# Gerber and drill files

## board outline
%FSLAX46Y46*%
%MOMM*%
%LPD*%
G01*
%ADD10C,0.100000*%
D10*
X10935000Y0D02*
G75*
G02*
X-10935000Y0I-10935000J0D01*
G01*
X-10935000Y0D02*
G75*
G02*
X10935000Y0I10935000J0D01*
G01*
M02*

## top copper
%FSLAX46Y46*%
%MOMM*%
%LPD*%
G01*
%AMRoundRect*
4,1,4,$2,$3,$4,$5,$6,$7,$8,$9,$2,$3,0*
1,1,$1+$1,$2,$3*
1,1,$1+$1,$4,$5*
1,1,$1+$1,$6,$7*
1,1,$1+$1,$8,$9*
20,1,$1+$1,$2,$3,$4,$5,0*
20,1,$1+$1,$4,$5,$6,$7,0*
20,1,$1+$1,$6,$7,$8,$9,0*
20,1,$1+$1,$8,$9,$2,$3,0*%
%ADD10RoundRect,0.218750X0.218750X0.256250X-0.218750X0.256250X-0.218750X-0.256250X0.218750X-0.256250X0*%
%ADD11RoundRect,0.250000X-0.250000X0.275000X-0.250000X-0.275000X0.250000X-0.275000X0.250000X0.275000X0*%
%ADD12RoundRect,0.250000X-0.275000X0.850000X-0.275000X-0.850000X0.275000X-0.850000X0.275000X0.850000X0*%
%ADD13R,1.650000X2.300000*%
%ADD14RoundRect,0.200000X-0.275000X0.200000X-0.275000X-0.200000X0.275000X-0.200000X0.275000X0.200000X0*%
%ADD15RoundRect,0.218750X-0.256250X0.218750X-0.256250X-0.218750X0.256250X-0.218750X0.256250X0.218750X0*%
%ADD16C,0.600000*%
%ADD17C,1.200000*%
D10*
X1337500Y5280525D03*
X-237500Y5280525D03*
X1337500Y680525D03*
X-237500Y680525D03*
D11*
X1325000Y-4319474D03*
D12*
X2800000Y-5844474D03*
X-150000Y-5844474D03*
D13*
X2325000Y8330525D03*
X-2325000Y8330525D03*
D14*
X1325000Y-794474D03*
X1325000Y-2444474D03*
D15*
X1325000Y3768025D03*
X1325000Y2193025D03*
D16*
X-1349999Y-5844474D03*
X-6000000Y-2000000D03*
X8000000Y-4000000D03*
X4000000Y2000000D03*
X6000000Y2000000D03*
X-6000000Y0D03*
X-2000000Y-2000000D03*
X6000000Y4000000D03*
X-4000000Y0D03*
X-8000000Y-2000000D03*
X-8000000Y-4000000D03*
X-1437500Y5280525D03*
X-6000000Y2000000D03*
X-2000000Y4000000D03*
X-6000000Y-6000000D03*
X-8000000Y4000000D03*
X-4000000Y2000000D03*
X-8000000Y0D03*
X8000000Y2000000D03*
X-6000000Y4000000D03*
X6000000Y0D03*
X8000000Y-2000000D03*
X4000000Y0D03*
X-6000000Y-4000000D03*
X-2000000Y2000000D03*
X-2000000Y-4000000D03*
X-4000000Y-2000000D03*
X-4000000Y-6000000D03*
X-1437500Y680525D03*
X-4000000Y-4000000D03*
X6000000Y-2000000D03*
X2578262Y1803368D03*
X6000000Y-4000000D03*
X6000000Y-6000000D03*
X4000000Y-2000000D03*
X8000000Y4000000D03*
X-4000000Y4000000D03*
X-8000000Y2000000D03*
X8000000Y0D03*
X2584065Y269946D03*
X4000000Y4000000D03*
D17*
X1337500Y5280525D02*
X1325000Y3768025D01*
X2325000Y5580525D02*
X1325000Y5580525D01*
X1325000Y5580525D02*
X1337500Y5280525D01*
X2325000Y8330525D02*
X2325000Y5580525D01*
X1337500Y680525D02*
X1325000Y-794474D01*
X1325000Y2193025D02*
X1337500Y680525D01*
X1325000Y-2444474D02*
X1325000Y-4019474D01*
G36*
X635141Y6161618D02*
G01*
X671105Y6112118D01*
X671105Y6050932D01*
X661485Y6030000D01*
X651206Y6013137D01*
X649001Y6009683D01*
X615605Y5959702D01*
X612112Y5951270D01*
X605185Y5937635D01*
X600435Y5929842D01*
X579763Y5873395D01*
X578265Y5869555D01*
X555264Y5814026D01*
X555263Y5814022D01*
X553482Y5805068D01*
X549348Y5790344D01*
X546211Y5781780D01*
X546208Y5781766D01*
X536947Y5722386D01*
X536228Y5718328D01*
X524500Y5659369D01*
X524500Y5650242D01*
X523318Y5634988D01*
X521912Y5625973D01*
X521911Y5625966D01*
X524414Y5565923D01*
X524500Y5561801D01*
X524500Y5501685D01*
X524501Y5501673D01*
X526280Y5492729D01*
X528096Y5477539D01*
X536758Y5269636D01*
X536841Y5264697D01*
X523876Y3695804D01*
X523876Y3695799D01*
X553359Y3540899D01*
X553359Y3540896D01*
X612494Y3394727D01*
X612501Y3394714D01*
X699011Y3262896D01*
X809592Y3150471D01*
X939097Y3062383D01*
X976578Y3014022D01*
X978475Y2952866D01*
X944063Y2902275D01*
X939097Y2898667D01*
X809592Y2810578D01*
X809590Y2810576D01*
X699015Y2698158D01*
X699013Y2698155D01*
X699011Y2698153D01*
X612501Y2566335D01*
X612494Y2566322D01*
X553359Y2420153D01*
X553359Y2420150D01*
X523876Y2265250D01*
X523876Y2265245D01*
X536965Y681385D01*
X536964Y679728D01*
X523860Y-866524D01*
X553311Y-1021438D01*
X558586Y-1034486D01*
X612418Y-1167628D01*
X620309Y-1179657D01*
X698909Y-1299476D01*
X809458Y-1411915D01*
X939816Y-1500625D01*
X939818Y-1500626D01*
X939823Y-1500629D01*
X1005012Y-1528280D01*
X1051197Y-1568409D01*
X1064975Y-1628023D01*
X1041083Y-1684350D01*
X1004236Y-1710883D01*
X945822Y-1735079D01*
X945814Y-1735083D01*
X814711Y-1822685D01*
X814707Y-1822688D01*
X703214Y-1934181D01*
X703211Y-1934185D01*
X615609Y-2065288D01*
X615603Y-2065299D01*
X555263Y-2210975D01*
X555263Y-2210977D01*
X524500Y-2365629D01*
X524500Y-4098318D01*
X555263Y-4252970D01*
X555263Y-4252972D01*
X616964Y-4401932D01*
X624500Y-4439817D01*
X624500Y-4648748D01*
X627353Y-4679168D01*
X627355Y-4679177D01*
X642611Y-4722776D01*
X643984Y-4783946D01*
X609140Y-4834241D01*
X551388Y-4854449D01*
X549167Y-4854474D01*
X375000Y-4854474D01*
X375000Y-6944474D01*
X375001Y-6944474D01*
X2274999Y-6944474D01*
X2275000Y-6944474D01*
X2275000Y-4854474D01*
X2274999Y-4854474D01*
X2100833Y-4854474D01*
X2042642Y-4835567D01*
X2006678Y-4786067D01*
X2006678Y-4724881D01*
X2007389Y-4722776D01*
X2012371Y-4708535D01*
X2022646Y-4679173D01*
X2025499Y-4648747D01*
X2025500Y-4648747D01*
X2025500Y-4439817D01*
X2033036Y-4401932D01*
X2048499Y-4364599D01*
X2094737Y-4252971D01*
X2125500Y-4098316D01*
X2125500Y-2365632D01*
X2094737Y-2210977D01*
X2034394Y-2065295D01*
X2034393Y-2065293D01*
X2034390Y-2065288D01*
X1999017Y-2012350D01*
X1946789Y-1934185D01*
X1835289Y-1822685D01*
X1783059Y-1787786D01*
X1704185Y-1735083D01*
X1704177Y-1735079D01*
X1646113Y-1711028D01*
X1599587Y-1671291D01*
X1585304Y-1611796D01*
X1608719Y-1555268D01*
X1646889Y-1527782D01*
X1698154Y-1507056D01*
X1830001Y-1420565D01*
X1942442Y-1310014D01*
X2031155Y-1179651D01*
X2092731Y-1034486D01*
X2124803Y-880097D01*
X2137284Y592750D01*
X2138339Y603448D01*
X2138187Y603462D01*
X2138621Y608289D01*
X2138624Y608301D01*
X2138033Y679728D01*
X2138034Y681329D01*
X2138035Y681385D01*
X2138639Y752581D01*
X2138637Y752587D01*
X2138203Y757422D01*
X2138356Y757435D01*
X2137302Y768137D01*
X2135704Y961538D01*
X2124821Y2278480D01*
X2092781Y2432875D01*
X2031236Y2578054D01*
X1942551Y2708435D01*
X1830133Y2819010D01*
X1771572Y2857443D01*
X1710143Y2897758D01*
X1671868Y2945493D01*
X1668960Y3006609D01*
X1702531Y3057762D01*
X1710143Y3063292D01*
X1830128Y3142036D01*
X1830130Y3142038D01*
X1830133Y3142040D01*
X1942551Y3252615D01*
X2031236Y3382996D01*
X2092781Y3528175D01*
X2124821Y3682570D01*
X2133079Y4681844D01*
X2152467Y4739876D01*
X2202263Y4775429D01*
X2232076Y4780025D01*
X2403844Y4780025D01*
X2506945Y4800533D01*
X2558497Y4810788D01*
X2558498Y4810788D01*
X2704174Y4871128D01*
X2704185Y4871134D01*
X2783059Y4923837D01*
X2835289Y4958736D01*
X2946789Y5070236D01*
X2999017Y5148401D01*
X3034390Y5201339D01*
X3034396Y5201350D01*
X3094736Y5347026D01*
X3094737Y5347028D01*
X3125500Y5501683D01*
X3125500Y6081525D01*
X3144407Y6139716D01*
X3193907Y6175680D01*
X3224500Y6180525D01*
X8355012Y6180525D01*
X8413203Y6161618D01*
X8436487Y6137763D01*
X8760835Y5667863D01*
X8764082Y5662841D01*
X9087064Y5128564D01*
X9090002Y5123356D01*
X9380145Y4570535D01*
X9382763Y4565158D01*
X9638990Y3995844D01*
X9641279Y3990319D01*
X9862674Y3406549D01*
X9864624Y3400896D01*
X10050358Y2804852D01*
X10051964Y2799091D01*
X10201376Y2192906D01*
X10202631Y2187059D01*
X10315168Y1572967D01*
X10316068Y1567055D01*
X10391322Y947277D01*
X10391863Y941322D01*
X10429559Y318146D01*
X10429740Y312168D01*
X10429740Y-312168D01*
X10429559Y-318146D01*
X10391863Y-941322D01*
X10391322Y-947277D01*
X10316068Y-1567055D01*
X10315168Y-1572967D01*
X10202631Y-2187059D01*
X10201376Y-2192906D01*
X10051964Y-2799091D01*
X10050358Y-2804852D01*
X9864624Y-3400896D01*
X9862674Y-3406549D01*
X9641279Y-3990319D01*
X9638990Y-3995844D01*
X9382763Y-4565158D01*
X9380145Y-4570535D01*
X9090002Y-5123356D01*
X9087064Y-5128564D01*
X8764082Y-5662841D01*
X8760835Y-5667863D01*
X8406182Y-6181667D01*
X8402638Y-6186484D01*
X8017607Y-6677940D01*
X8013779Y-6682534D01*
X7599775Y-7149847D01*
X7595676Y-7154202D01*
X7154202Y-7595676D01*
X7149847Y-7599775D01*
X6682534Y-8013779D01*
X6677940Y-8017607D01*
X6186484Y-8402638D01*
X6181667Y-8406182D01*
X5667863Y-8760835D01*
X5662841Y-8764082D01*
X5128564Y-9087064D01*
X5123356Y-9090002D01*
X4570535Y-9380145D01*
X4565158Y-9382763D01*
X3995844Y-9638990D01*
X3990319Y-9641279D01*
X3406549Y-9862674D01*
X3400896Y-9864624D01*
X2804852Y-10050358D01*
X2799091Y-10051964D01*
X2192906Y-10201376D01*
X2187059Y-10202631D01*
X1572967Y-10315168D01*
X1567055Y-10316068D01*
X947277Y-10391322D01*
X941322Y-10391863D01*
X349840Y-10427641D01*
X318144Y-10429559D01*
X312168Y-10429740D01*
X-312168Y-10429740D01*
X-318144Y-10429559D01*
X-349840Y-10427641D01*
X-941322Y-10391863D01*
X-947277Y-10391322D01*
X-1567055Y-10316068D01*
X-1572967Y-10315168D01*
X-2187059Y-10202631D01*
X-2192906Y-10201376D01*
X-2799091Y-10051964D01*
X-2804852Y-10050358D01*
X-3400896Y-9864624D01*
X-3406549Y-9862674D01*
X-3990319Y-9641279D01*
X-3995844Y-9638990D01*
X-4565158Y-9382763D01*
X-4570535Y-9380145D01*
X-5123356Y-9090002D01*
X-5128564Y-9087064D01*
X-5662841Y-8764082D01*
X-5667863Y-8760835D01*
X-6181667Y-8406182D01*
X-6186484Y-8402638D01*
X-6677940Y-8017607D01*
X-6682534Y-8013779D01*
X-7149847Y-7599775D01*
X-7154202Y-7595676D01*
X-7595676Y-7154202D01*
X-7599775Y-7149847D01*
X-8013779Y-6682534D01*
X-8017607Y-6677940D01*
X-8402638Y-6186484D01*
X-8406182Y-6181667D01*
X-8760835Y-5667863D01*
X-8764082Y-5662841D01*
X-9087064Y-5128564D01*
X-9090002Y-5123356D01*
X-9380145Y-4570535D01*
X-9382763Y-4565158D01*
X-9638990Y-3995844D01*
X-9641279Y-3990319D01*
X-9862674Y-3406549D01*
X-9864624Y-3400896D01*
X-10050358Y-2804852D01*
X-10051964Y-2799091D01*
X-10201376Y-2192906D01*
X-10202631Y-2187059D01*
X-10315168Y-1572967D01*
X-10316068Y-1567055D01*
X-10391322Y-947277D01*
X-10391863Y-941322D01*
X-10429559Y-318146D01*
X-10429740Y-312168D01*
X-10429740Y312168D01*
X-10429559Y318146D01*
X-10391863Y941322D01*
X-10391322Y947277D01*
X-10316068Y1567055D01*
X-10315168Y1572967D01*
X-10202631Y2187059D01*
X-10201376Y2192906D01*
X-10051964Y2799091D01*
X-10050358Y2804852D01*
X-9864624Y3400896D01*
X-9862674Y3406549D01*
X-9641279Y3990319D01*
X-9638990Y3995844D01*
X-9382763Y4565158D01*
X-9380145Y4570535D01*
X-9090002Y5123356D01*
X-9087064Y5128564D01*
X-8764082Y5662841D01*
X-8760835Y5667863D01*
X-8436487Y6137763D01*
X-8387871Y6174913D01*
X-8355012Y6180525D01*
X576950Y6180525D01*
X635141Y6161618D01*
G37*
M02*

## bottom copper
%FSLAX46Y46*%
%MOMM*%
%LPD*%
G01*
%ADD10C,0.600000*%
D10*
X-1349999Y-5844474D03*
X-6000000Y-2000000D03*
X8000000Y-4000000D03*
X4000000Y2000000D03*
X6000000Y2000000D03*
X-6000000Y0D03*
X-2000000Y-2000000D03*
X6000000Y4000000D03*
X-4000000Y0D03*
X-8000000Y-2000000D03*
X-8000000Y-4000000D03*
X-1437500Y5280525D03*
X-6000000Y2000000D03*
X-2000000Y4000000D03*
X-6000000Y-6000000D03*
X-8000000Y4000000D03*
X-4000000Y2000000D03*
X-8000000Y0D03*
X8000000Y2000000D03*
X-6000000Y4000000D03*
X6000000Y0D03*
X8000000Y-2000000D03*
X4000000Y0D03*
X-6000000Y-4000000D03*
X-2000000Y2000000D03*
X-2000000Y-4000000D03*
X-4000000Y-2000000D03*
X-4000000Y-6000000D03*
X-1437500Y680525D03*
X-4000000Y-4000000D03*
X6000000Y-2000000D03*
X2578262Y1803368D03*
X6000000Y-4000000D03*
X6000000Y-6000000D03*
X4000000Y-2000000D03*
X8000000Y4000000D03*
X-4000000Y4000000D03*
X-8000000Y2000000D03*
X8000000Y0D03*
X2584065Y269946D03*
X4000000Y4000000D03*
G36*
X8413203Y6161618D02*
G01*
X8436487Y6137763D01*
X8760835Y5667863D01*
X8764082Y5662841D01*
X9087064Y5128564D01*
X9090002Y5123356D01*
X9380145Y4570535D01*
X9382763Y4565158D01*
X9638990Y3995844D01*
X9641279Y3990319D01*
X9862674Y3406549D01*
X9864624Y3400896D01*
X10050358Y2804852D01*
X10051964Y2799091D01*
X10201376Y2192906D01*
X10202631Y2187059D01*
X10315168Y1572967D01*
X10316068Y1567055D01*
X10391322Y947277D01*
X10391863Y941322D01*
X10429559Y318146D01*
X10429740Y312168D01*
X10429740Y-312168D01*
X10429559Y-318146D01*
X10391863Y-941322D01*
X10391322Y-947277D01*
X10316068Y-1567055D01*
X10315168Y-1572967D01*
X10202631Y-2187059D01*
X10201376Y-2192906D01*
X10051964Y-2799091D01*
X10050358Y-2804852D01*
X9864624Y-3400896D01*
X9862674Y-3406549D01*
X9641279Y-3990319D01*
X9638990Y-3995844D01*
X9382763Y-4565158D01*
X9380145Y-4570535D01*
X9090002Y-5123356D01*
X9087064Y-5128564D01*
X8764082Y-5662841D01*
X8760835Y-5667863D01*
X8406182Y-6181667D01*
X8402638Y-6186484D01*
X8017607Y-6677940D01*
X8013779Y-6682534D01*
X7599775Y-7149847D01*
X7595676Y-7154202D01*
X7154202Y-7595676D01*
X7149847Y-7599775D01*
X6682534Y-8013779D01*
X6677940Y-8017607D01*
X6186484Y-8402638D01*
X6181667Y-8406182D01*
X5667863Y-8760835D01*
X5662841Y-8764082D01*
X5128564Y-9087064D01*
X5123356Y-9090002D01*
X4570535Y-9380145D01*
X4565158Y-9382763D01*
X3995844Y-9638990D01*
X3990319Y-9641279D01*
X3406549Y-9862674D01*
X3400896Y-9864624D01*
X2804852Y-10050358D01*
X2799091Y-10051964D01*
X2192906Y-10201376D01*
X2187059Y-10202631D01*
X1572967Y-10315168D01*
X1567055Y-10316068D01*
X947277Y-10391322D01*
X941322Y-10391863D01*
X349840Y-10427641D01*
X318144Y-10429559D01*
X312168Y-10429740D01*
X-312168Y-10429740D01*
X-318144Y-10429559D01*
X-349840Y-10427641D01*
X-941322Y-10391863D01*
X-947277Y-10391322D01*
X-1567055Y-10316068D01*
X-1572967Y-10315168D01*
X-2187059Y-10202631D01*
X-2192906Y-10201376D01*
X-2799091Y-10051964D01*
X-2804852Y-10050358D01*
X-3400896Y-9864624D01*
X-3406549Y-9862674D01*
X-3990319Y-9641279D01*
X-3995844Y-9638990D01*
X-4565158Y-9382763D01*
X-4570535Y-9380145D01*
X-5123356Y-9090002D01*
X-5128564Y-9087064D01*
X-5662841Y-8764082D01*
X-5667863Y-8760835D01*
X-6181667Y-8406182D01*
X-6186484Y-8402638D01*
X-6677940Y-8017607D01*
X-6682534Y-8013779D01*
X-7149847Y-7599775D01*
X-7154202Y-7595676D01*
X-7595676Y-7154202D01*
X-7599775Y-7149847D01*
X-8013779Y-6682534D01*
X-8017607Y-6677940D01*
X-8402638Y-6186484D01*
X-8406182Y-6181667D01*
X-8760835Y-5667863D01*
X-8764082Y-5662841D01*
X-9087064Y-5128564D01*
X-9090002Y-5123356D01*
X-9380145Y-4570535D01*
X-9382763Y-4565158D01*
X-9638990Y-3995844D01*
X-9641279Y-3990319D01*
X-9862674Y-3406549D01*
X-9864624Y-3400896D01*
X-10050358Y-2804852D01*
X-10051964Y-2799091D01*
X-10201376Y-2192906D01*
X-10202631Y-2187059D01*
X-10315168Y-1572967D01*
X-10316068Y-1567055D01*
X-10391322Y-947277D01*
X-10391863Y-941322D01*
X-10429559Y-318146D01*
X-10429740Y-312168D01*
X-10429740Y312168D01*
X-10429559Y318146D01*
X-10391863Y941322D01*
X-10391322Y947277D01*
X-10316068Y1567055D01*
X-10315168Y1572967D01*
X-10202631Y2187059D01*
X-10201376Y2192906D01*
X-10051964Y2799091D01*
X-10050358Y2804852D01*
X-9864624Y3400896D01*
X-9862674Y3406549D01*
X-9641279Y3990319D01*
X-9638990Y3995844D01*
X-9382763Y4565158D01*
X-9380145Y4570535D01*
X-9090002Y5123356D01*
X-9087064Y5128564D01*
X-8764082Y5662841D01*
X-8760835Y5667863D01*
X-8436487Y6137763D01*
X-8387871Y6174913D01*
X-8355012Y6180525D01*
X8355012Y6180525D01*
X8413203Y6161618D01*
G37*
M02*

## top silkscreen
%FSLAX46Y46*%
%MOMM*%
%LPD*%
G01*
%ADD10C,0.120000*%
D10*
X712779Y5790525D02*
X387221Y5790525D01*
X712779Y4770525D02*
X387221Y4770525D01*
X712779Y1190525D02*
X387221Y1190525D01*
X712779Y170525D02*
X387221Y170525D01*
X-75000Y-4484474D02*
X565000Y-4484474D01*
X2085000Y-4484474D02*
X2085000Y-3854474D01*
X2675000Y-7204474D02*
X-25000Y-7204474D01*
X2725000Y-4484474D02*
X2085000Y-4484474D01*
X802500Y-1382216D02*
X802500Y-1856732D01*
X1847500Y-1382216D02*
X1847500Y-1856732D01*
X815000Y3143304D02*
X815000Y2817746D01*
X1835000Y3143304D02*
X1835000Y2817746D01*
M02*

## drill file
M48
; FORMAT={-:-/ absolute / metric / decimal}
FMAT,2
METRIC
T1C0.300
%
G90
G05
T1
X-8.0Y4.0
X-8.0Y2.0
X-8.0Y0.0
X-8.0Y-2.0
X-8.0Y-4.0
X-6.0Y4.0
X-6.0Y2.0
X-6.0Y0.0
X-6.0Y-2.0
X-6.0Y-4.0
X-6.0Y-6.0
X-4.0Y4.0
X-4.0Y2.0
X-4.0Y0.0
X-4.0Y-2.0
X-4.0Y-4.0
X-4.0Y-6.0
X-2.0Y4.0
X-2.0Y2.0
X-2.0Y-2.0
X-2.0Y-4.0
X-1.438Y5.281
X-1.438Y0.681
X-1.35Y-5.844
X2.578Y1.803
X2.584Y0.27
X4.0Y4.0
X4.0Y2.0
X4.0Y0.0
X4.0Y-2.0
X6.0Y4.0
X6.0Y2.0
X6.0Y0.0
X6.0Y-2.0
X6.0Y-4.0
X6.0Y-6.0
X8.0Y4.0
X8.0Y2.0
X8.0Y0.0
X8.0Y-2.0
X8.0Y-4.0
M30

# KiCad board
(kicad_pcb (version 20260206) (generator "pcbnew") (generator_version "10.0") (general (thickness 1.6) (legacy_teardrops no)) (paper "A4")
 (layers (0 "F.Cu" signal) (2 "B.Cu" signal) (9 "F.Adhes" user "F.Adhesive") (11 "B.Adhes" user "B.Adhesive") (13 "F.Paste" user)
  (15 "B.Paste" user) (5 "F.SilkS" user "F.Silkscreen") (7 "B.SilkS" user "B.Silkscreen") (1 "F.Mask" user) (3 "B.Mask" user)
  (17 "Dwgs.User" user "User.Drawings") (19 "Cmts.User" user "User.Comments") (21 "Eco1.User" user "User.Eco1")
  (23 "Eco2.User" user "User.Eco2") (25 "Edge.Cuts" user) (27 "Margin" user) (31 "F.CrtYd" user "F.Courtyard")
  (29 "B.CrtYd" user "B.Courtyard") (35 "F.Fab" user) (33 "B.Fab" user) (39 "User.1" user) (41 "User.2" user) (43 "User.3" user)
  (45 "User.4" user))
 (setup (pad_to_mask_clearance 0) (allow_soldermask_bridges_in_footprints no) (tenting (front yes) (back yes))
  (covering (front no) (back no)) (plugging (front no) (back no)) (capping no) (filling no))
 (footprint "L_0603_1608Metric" (layer "F.Cu") (at 0.55 -5.280525 180)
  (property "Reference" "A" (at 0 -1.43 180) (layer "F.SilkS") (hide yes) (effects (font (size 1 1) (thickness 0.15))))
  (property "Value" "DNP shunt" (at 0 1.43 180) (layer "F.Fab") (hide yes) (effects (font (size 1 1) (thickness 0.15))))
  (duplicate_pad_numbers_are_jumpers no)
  (fp_line (start -0.162779 0.51) (end 0.162779 0.51) (stroke (width 0.12) (type solid)) (layer "F.SilkS"))
  (fp_line (start -0.162779 -0.51) (end 0.162779 -0.51) (stroke (width 0.12) (type solid)) (layer "F.SilkS"))
  (pad "1" smd roundrect (at -0.7875 0 180) (size 0.875 0.95) (layers "F.Cu" "F.Mask" "F.Paste") (roundrect_rratio 0.25) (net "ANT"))
  (pad "2" smd roundrect (at 0.7875 0 180) (size 0.875 0.95) (layers "F.Cu" "F.Mask" "F.Paste") (roundrect_rratio 0.25) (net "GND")))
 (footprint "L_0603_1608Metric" (layer "F.Cu") (at 0.55 -0.680525 180)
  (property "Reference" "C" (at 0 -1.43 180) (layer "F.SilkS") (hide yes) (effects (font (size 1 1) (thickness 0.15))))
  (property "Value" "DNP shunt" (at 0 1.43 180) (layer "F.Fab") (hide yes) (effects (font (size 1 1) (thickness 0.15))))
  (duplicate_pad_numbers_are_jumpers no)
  (fp_line (start -0.162779 0.51) (end 0.162779 0.51) (stroke (width 0.12) (type solid)) (layer "F.SilkS"))
  (fp_line (start -0.162779 -0.51) (end 0.162779 -0.51) (stroke (width 0.12) (type solid)) (layer "F.SilkS"))
  (pad "1" smd roundrect (at -0.7875 0 180) (size 0.875 0.95) (layers "F.Cu" "F.Mask" "F.Paste") (roundrect_rratio 0.25) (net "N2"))
  (pad "2" smd roundrect (at 0.7875 0 180) (size 0.875 0.95) (layers "F.Cu" "F.Mask" "F.Paste") (roundrect_rratio 0.25) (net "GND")))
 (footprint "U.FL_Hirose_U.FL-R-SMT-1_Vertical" (layer "F.Cu") (at 1.325 5.844474 -90)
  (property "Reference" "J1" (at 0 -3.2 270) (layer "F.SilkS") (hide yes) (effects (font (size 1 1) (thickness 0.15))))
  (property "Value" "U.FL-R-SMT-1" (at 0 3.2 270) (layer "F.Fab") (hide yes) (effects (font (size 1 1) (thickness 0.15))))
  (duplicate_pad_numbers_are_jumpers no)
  (fp_line (start -1.36 1.4) (end -1.36 0.76) (stroke (width 0.12) (type solid)) (layer "F.SilkS"))
  (fp_line (start -1.36 -0.76) (end -1.99 -0.76) (stroke (width 0.12) (type solid)) (layer "F.SilkS"))
  (fp_line (start 1.36 -1.35) (end 1.36 1.35) (stroke (width 0.12) (type solid)) (layer "F.SilkS"))
  (fp_line (start -1.36 -1.4) (end -1.36 -0.76) (stroke (width 0.12) (type solid)) (layer "F.SilkS"))
  (pad "1" smd roundrect (at -1.525 0 270) (size 1.05 1) (layers "F.Cu" "F.Mask" "F.Paste") (roundrect_rratio 0.25) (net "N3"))
  (pad "2" smd roundrect (at 0 -1.475 270) (size 2.2 1.05) (layers "F.Cu" "F.Mask" "F.Paste") (roundrect_rratio 0.2380952381) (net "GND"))
  (pad "2" smd roundrect (at 0 1.475 270) (size 2.2 1.05) (layers "F.Cu" "F.Mask" "F.Paste") (roundrect_rratio 0.2380952381) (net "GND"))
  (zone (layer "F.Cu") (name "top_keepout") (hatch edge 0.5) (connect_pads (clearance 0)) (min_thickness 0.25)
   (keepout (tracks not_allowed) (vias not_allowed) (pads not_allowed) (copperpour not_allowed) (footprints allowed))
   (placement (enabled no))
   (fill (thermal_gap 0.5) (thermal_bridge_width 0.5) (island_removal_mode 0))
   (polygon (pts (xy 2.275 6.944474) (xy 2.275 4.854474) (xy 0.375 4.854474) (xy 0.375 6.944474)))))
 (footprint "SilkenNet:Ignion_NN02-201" (layer "F.Cu") (at 0 -8.330525)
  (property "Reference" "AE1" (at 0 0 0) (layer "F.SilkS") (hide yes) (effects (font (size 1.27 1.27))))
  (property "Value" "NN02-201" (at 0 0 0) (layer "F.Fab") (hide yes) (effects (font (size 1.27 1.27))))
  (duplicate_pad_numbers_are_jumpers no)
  (pad "1" smd rect (at 2.325 0) (size 1.65 2.3) (layers "F.Cu" "F.Mask" "F.Paste") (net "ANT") (thermal_bridge_angle 45))
  (pad "2" smd rect (at -2.325 0) (size 1.65 2.3) (layers "F.Cu" "F.Mask" "F.Paste") (thermal_bridge_angle 45)))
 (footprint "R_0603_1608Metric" (layer "F.Cu") (at 1.325 1.619474 -90)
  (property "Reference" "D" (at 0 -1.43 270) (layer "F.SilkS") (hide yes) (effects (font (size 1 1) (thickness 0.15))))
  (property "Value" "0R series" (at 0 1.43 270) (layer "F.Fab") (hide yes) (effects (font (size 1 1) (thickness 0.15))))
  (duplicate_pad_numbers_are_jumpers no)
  (fp_line (start -0.237258 0.5225) (end 0.237258 0.5225) (stroke (width 0.12) (type solid)) (layer "F.SilkS"))
  (fp_line (start -0.237258 -0.5225) (end 0.237258 -0.5225) (stroke (width 0.12) (type solid)) (layer "F.SilkS"))
  (pad "1" smd roundrect (at -0.825 0 270) (size 0.8 0.95) (layers "F.Cu" "F.Mask" "F.Paste") (roundrect_rratio 0.25) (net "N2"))
  (pad "2" smd roundrect (at 0.825 0 270) (size 0.8 0.95) (layers "F.Cu" "F.Mask" "F.Paste") (roundrect_rratio 0.25) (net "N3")))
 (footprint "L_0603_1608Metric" (layer "F.Cu") (at 1.325 -2.980525 -90)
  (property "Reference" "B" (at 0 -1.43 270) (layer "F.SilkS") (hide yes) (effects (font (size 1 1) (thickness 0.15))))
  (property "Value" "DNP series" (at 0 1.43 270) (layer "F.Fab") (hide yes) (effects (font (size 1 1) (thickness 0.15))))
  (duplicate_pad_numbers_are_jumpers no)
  (fp_line (start -0.162779 0.51) (end 0.162779 0.51) (stroke (width 0.12) (type solid)) (layer "F.SilkS"))
  (fp_line (start -0.162779 -0.51) (end 0.162779 -0.51) (stroke (width 0.12) (type solid)) (layer "F.SilkS"))
  (pad "1" smd roundrect (at -0.7875 0 270) (size 0.875 0.95) (layers "F.Cu" "F.Mask" "F.Paste") (roundrect_rratio 0.25) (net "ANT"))
  (pad "2" smd roundrect (at 0.7875 0 270) (size 0.875 0.95) (layers "F.Cu" "F.Mask" "F.Paste") (roundrect_rratio 0.25) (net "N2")))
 (gr_circle (center 0 0) (end 10.935 0) (stroke (width 0.1) (type default)) (fill no) (layer "Edge.Cuts"))
 (via (at -1.349999 5.844474) (size 0.6) (drill 0.3) (layers "F.Cu" "B.Cu") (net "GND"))
 (via (at -6 2) (size 0.6) (drill 0.3) (layers "F.Cu" "B.Cu") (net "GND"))
 (via (at 8 4) (size 0.6) (drill 0.3) (layers "F.Cu" "B.Cu") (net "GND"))
 (via (at 4 -2) (size 0.6) (drill 0.3) (layers "F.Cu" "B.Cu") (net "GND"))
 (via (at 6 -2) (size 0.6) (drill 0.3) (layers "F.Cu" "B.Cu") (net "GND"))
 (via (at -6 0) (size 0.6) (drill 0.3) (layers "F.Cu" "B.Cu") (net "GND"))
 (via (at -2 2) (size 0.6) (drill 0.3) (layers "F.Cu" "B.Cu") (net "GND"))
 (via (at 6 -4) (size 0.6) (drill 0.3) (layers "F.Cu" "B.Cu") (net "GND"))
 (via (at -4 0) (size 0.6) (drill 0.3) (layers "F.Cu" "B.Cu") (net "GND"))
 (via (at -8 2) (size 0.6) (drill 0.3) (layers "F.Cu" "B.Cu") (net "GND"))
 (via (at -8 4) (size 0.6) (drill 0.3) (layers "F.Cu" "B.Cu") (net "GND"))
 (via (at -1.4375 -5.280525) (size 0.6) (drill 0.3) (layers "F.Cu" "B.Cu") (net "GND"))
 (via (at -6 -2) (size 0.6) (drill 0.3) (layers "F.Cu" "B.Cu") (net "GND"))
 (via (at -2 -4) (size 0.6) (drill 0.3) (layers "F.Cu" "B.Cu") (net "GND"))
 (via (at -6 6) (size 0.6) (drill 0.3) (layers "F.Cu" "B.Cu") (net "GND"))
 (via (at -8 -4) (size 0.6) (drill 0.3) (layers "F.Cu" "B.Cu") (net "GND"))
 (via (at -4 -2) (size 0.6) (drill 0.3) (layers "F.Cu" "B.Cu") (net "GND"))
 (via (at -8 0) (size 0.6) (drill 0.3) (layers "F.Cu" "B.Cu") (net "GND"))
 (via (at 8 -2) (size 0.6) (drill 0.3) (layers "F.Cu" "B.Cu") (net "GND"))
 (via (at -6 -4) (size 0.6) (drill 0.3) (layers "F.Cu" "B.Cu") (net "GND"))
 (via (at 6 0) (size 0.6) (drill 0.3) (layers "F.Cu" "B.Cu") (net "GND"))
 (via (at 8 2) (size 0.6) (drill 0.3) (layers "F.Cu" "B.Cu") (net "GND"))
 (via (at 4 0) (size 0.6) (drill 0.3) (layers "F.Cu" "B.Cu") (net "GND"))
 (via (at -6 4) (size 0.6) (drill 0.3) (layers "F.Cu" "B.Cu") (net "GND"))
 (via (at -2 -2) (size 0.6) (drill 0.3) (layers "F.Cu" "B.Cu") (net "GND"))
 (via (at -2 4) (size 0.6) (drill 0.3) (layers "F.Cu" "B.Cu") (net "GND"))
 (via (at -4 2) (size 0.6) (drill 0.3) (layers "F.Cu" "B.Cu") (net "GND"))
 (via (at -4 6) (size 0.6) (drill 0.3) (layers "F.Cu" "B.Cu") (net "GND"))
 (via (at -1.4375 -0.680525) (size 0.6) (drill 0.3) (layers "F.Cu" "B.Cu") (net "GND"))
 (via (at -4 4) (size 0.6) (drill 0.3) (layers "F.Cu" "B.Cu") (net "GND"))
 (via (at 6 2) (size 0.6) (drill 0.3) (layers "F.Cu" "B.Cu") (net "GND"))
 (via (at 2.578262 -1.803368) (size 0.6) (drill 0.3) (layers "F.Cu" "B.Cu") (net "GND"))
 (via (at 6 4) (size 0.6) (drill 0.3) (layers "F.Cu" "B.Cu") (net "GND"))
 (via (at 6 6) (size 0.6) (drill 0.3) (layers "F.Cu" "B.Cu") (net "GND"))
 (via (at 4 2) (size 0.6) (drill 0.3) (layers "F.Cu" "B.Cu") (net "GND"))
 (via (at 8 -4) (size 0.6) (drill 0.3) (layers "F.Cu" "B.Cu") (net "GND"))
 (via (at -4 -4) (size 0.6) (drill 0.3) (layers "F.Cu" "B.Cu") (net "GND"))
 (via (at -8 -2) (size 0.6) (drill 0.3) (layers "F.Cu" "B.Cu") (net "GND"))
 (via (at 8 0) (size 0.6) (drill 0.3) (layers "F.Cu" "B.Cu") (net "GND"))
 (via (at 2.584065 -0.269946) (size 0.6) (drill 0.3) (layers "F.Cu" "B.Cu") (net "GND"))
 (via (at 4 -4) (size 0.6) (drill 0.3) (layers "F.Cu" "B.Cu") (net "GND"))
 (segment (start 1.3375 -5.280525) (end 1.325 -3.768025) (width 1.2) (layer "F.Cu") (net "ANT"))
 (segment (start 2.325 -5.580525) (end 1.325 -5.580525) (width 1.2) (layer "F.Cu") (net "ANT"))
 (segment (start 1.325 -5.580525) (end 1.3375 -5.280525) (width 1.2) (layer "F.Cu") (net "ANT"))
 (segment (start 2.325 -8.330525) (end 2.325 -5.580525) (width 1.2) (layer "F.Cu") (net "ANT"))
 (segment (start 1.3375 -0.680525) (end 1.325 0.794474) (width 1.2) (layer "F.Cu") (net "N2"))
 (segment (start 1.325 -2.193025) (end 1.3375 -0.680525) (width 1.2) (layer "F.Cu") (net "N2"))
 (segment (start 1.325 2.444474) (end 1.325 4.019474) (width 1.2) (layer "F.Cu") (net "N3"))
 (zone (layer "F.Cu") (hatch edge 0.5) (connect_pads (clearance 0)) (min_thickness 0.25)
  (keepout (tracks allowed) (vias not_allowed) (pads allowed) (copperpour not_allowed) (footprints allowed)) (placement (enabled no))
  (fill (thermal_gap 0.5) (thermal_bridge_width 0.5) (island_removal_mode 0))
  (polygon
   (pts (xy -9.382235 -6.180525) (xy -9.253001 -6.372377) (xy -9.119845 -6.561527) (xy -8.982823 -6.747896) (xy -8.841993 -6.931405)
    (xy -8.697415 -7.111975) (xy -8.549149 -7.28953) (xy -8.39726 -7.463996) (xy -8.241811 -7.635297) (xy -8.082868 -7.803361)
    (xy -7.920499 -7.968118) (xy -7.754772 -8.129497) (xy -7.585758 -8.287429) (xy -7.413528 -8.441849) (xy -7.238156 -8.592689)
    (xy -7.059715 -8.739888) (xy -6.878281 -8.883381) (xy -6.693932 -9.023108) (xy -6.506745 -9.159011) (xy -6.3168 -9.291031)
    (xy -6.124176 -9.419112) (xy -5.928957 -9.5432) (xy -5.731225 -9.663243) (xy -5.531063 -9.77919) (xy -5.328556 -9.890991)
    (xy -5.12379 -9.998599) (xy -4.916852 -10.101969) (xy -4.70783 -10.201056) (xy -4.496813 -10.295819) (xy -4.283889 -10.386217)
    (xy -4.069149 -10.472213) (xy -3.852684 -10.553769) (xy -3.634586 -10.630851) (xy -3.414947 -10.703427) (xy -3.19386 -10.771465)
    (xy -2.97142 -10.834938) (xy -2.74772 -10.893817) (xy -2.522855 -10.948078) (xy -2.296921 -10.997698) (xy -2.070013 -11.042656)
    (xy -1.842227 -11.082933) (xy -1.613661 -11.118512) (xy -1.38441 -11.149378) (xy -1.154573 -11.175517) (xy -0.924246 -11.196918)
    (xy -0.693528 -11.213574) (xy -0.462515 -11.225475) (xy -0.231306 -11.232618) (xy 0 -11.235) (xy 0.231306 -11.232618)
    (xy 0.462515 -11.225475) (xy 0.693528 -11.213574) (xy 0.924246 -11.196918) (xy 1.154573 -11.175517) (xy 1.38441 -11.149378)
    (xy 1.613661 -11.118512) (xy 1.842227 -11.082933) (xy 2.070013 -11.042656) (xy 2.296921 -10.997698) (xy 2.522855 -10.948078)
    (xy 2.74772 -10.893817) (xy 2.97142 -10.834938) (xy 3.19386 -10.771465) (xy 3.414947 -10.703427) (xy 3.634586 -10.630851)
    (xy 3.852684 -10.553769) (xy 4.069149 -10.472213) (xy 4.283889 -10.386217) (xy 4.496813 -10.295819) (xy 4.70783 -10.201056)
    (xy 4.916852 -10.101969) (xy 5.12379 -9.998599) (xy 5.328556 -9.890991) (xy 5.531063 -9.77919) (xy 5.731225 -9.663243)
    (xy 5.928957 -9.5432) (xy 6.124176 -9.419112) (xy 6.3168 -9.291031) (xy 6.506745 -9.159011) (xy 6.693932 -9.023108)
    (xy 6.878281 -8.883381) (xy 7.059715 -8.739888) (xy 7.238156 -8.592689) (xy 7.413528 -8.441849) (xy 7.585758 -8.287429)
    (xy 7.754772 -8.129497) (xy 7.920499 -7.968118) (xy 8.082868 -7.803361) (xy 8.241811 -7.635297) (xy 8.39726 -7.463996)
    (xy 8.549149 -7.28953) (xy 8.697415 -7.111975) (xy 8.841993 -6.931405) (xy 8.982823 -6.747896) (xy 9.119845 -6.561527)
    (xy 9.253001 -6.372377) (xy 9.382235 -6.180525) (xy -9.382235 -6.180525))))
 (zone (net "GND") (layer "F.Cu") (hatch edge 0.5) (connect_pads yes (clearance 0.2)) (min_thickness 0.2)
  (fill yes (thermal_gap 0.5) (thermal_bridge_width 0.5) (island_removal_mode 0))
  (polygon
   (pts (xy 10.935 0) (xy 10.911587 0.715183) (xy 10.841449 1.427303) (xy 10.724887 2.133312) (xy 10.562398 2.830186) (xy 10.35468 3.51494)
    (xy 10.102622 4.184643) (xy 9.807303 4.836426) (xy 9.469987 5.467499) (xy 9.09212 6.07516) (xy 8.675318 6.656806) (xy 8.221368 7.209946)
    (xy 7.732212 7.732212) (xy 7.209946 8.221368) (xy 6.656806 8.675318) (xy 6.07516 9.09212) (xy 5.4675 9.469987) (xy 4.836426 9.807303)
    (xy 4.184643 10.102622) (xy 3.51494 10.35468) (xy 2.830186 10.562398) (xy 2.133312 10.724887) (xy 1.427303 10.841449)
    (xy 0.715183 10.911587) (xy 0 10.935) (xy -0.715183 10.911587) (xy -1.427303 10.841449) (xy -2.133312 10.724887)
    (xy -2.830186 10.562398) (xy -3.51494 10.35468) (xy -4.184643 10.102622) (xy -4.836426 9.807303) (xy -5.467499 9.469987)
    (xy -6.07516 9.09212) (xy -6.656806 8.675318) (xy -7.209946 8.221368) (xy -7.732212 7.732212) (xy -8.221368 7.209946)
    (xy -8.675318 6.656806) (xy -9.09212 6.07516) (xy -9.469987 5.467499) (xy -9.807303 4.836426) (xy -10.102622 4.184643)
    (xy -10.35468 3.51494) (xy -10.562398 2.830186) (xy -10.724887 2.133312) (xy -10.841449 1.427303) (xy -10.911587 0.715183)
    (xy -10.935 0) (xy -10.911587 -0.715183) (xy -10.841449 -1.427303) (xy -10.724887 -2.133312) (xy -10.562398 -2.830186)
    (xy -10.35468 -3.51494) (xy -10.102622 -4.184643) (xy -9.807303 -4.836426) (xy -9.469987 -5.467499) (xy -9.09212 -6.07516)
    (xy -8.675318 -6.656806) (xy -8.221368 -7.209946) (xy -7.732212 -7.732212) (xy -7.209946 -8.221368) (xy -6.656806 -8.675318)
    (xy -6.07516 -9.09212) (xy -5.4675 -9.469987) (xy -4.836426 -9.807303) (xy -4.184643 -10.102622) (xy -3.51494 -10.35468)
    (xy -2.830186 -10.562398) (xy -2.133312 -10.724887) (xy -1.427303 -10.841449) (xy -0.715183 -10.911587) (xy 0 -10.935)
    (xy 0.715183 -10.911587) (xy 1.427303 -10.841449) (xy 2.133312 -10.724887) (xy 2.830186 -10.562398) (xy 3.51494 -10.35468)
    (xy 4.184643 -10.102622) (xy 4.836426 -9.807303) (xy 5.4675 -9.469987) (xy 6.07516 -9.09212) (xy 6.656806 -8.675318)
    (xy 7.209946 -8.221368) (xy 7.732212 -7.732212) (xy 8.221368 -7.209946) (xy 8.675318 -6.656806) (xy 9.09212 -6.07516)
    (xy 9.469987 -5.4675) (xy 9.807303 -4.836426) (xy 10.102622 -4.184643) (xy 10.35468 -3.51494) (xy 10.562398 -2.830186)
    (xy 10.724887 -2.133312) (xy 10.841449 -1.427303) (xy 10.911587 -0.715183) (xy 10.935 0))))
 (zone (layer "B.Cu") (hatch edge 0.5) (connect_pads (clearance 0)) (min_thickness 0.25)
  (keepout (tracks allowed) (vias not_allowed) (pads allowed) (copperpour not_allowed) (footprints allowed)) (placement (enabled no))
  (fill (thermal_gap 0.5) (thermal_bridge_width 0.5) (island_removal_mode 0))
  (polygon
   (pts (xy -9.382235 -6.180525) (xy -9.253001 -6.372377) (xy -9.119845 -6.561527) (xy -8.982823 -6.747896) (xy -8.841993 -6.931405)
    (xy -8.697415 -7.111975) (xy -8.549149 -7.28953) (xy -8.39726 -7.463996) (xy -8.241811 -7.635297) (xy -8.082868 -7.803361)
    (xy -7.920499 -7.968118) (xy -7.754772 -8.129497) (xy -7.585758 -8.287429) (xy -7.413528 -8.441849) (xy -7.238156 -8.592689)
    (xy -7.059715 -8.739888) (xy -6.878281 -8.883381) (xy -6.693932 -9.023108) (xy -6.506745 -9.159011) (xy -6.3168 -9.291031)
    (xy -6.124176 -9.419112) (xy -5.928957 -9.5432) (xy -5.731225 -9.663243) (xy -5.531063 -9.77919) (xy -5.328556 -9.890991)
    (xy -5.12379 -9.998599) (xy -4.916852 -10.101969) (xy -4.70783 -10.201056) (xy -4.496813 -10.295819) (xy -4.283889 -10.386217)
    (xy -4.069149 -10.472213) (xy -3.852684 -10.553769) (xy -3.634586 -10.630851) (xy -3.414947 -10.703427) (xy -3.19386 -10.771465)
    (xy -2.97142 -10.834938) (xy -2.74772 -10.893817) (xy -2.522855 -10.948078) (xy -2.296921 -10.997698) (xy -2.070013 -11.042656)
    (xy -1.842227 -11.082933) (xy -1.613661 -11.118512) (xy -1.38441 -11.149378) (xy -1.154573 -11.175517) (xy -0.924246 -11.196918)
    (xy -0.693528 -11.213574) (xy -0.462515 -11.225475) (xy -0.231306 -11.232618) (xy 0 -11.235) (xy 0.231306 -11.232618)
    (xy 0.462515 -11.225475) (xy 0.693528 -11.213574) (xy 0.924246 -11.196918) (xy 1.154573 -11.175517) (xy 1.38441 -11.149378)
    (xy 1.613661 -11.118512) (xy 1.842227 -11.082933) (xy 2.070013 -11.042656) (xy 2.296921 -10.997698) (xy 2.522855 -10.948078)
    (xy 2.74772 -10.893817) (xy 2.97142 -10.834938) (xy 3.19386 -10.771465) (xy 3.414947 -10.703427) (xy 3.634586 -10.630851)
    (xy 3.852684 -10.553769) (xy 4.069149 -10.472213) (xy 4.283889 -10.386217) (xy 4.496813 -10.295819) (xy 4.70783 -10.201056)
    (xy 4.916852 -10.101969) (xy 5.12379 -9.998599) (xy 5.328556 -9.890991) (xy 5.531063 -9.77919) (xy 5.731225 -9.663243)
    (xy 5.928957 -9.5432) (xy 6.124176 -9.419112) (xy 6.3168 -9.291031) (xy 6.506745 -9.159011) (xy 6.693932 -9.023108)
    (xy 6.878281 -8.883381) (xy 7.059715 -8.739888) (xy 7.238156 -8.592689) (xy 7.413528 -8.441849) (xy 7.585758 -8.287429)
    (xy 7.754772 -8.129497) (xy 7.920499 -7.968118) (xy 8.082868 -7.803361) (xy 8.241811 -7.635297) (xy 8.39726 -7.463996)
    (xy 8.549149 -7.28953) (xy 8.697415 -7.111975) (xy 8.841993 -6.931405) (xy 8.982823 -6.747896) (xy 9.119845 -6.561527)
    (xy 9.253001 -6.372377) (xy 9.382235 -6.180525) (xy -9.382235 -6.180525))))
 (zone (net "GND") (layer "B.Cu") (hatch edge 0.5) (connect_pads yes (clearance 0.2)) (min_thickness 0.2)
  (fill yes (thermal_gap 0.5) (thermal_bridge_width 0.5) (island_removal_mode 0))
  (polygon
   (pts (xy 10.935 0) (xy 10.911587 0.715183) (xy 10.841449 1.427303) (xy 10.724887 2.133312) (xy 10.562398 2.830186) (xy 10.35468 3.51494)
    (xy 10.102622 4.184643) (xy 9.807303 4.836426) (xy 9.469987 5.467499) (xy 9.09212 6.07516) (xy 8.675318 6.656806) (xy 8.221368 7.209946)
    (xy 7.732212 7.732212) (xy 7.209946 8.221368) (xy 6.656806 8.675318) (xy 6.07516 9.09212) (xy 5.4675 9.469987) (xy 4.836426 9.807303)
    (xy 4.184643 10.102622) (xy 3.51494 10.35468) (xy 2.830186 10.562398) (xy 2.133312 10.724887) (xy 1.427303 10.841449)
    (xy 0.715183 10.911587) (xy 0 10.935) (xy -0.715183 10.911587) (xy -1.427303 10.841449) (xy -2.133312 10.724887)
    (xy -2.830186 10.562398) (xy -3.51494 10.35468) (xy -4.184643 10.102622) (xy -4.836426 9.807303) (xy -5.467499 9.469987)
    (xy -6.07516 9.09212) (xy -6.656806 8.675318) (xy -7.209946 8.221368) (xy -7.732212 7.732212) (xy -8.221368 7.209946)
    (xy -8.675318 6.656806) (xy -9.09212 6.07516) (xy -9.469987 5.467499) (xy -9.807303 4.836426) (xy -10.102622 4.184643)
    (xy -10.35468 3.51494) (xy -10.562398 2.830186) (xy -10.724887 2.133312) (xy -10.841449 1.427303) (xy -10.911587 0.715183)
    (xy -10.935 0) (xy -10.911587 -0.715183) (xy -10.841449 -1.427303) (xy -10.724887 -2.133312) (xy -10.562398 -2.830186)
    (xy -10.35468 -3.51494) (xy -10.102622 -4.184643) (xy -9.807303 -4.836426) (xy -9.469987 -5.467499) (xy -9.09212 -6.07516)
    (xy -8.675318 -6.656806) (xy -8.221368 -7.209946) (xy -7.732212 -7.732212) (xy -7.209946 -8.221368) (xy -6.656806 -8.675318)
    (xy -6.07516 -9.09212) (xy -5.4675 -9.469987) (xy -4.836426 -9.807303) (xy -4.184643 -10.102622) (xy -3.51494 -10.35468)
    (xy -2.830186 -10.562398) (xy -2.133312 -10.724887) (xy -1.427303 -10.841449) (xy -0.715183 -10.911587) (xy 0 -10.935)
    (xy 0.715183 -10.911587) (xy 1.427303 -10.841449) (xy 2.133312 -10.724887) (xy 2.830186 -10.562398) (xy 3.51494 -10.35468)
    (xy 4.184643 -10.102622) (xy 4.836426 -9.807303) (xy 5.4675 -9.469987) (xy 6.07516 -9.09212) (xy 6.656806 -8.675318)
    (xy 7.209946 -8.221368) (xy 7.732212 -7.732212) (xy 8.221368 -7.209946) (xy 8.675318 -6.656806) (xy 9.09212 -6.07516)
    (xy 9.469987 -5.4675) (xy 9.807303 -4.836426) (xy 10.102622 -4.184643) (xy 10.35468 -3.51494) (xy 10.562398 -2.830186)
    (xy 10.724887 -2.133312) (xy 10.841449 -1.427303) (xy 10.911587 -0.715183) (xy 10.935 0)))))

